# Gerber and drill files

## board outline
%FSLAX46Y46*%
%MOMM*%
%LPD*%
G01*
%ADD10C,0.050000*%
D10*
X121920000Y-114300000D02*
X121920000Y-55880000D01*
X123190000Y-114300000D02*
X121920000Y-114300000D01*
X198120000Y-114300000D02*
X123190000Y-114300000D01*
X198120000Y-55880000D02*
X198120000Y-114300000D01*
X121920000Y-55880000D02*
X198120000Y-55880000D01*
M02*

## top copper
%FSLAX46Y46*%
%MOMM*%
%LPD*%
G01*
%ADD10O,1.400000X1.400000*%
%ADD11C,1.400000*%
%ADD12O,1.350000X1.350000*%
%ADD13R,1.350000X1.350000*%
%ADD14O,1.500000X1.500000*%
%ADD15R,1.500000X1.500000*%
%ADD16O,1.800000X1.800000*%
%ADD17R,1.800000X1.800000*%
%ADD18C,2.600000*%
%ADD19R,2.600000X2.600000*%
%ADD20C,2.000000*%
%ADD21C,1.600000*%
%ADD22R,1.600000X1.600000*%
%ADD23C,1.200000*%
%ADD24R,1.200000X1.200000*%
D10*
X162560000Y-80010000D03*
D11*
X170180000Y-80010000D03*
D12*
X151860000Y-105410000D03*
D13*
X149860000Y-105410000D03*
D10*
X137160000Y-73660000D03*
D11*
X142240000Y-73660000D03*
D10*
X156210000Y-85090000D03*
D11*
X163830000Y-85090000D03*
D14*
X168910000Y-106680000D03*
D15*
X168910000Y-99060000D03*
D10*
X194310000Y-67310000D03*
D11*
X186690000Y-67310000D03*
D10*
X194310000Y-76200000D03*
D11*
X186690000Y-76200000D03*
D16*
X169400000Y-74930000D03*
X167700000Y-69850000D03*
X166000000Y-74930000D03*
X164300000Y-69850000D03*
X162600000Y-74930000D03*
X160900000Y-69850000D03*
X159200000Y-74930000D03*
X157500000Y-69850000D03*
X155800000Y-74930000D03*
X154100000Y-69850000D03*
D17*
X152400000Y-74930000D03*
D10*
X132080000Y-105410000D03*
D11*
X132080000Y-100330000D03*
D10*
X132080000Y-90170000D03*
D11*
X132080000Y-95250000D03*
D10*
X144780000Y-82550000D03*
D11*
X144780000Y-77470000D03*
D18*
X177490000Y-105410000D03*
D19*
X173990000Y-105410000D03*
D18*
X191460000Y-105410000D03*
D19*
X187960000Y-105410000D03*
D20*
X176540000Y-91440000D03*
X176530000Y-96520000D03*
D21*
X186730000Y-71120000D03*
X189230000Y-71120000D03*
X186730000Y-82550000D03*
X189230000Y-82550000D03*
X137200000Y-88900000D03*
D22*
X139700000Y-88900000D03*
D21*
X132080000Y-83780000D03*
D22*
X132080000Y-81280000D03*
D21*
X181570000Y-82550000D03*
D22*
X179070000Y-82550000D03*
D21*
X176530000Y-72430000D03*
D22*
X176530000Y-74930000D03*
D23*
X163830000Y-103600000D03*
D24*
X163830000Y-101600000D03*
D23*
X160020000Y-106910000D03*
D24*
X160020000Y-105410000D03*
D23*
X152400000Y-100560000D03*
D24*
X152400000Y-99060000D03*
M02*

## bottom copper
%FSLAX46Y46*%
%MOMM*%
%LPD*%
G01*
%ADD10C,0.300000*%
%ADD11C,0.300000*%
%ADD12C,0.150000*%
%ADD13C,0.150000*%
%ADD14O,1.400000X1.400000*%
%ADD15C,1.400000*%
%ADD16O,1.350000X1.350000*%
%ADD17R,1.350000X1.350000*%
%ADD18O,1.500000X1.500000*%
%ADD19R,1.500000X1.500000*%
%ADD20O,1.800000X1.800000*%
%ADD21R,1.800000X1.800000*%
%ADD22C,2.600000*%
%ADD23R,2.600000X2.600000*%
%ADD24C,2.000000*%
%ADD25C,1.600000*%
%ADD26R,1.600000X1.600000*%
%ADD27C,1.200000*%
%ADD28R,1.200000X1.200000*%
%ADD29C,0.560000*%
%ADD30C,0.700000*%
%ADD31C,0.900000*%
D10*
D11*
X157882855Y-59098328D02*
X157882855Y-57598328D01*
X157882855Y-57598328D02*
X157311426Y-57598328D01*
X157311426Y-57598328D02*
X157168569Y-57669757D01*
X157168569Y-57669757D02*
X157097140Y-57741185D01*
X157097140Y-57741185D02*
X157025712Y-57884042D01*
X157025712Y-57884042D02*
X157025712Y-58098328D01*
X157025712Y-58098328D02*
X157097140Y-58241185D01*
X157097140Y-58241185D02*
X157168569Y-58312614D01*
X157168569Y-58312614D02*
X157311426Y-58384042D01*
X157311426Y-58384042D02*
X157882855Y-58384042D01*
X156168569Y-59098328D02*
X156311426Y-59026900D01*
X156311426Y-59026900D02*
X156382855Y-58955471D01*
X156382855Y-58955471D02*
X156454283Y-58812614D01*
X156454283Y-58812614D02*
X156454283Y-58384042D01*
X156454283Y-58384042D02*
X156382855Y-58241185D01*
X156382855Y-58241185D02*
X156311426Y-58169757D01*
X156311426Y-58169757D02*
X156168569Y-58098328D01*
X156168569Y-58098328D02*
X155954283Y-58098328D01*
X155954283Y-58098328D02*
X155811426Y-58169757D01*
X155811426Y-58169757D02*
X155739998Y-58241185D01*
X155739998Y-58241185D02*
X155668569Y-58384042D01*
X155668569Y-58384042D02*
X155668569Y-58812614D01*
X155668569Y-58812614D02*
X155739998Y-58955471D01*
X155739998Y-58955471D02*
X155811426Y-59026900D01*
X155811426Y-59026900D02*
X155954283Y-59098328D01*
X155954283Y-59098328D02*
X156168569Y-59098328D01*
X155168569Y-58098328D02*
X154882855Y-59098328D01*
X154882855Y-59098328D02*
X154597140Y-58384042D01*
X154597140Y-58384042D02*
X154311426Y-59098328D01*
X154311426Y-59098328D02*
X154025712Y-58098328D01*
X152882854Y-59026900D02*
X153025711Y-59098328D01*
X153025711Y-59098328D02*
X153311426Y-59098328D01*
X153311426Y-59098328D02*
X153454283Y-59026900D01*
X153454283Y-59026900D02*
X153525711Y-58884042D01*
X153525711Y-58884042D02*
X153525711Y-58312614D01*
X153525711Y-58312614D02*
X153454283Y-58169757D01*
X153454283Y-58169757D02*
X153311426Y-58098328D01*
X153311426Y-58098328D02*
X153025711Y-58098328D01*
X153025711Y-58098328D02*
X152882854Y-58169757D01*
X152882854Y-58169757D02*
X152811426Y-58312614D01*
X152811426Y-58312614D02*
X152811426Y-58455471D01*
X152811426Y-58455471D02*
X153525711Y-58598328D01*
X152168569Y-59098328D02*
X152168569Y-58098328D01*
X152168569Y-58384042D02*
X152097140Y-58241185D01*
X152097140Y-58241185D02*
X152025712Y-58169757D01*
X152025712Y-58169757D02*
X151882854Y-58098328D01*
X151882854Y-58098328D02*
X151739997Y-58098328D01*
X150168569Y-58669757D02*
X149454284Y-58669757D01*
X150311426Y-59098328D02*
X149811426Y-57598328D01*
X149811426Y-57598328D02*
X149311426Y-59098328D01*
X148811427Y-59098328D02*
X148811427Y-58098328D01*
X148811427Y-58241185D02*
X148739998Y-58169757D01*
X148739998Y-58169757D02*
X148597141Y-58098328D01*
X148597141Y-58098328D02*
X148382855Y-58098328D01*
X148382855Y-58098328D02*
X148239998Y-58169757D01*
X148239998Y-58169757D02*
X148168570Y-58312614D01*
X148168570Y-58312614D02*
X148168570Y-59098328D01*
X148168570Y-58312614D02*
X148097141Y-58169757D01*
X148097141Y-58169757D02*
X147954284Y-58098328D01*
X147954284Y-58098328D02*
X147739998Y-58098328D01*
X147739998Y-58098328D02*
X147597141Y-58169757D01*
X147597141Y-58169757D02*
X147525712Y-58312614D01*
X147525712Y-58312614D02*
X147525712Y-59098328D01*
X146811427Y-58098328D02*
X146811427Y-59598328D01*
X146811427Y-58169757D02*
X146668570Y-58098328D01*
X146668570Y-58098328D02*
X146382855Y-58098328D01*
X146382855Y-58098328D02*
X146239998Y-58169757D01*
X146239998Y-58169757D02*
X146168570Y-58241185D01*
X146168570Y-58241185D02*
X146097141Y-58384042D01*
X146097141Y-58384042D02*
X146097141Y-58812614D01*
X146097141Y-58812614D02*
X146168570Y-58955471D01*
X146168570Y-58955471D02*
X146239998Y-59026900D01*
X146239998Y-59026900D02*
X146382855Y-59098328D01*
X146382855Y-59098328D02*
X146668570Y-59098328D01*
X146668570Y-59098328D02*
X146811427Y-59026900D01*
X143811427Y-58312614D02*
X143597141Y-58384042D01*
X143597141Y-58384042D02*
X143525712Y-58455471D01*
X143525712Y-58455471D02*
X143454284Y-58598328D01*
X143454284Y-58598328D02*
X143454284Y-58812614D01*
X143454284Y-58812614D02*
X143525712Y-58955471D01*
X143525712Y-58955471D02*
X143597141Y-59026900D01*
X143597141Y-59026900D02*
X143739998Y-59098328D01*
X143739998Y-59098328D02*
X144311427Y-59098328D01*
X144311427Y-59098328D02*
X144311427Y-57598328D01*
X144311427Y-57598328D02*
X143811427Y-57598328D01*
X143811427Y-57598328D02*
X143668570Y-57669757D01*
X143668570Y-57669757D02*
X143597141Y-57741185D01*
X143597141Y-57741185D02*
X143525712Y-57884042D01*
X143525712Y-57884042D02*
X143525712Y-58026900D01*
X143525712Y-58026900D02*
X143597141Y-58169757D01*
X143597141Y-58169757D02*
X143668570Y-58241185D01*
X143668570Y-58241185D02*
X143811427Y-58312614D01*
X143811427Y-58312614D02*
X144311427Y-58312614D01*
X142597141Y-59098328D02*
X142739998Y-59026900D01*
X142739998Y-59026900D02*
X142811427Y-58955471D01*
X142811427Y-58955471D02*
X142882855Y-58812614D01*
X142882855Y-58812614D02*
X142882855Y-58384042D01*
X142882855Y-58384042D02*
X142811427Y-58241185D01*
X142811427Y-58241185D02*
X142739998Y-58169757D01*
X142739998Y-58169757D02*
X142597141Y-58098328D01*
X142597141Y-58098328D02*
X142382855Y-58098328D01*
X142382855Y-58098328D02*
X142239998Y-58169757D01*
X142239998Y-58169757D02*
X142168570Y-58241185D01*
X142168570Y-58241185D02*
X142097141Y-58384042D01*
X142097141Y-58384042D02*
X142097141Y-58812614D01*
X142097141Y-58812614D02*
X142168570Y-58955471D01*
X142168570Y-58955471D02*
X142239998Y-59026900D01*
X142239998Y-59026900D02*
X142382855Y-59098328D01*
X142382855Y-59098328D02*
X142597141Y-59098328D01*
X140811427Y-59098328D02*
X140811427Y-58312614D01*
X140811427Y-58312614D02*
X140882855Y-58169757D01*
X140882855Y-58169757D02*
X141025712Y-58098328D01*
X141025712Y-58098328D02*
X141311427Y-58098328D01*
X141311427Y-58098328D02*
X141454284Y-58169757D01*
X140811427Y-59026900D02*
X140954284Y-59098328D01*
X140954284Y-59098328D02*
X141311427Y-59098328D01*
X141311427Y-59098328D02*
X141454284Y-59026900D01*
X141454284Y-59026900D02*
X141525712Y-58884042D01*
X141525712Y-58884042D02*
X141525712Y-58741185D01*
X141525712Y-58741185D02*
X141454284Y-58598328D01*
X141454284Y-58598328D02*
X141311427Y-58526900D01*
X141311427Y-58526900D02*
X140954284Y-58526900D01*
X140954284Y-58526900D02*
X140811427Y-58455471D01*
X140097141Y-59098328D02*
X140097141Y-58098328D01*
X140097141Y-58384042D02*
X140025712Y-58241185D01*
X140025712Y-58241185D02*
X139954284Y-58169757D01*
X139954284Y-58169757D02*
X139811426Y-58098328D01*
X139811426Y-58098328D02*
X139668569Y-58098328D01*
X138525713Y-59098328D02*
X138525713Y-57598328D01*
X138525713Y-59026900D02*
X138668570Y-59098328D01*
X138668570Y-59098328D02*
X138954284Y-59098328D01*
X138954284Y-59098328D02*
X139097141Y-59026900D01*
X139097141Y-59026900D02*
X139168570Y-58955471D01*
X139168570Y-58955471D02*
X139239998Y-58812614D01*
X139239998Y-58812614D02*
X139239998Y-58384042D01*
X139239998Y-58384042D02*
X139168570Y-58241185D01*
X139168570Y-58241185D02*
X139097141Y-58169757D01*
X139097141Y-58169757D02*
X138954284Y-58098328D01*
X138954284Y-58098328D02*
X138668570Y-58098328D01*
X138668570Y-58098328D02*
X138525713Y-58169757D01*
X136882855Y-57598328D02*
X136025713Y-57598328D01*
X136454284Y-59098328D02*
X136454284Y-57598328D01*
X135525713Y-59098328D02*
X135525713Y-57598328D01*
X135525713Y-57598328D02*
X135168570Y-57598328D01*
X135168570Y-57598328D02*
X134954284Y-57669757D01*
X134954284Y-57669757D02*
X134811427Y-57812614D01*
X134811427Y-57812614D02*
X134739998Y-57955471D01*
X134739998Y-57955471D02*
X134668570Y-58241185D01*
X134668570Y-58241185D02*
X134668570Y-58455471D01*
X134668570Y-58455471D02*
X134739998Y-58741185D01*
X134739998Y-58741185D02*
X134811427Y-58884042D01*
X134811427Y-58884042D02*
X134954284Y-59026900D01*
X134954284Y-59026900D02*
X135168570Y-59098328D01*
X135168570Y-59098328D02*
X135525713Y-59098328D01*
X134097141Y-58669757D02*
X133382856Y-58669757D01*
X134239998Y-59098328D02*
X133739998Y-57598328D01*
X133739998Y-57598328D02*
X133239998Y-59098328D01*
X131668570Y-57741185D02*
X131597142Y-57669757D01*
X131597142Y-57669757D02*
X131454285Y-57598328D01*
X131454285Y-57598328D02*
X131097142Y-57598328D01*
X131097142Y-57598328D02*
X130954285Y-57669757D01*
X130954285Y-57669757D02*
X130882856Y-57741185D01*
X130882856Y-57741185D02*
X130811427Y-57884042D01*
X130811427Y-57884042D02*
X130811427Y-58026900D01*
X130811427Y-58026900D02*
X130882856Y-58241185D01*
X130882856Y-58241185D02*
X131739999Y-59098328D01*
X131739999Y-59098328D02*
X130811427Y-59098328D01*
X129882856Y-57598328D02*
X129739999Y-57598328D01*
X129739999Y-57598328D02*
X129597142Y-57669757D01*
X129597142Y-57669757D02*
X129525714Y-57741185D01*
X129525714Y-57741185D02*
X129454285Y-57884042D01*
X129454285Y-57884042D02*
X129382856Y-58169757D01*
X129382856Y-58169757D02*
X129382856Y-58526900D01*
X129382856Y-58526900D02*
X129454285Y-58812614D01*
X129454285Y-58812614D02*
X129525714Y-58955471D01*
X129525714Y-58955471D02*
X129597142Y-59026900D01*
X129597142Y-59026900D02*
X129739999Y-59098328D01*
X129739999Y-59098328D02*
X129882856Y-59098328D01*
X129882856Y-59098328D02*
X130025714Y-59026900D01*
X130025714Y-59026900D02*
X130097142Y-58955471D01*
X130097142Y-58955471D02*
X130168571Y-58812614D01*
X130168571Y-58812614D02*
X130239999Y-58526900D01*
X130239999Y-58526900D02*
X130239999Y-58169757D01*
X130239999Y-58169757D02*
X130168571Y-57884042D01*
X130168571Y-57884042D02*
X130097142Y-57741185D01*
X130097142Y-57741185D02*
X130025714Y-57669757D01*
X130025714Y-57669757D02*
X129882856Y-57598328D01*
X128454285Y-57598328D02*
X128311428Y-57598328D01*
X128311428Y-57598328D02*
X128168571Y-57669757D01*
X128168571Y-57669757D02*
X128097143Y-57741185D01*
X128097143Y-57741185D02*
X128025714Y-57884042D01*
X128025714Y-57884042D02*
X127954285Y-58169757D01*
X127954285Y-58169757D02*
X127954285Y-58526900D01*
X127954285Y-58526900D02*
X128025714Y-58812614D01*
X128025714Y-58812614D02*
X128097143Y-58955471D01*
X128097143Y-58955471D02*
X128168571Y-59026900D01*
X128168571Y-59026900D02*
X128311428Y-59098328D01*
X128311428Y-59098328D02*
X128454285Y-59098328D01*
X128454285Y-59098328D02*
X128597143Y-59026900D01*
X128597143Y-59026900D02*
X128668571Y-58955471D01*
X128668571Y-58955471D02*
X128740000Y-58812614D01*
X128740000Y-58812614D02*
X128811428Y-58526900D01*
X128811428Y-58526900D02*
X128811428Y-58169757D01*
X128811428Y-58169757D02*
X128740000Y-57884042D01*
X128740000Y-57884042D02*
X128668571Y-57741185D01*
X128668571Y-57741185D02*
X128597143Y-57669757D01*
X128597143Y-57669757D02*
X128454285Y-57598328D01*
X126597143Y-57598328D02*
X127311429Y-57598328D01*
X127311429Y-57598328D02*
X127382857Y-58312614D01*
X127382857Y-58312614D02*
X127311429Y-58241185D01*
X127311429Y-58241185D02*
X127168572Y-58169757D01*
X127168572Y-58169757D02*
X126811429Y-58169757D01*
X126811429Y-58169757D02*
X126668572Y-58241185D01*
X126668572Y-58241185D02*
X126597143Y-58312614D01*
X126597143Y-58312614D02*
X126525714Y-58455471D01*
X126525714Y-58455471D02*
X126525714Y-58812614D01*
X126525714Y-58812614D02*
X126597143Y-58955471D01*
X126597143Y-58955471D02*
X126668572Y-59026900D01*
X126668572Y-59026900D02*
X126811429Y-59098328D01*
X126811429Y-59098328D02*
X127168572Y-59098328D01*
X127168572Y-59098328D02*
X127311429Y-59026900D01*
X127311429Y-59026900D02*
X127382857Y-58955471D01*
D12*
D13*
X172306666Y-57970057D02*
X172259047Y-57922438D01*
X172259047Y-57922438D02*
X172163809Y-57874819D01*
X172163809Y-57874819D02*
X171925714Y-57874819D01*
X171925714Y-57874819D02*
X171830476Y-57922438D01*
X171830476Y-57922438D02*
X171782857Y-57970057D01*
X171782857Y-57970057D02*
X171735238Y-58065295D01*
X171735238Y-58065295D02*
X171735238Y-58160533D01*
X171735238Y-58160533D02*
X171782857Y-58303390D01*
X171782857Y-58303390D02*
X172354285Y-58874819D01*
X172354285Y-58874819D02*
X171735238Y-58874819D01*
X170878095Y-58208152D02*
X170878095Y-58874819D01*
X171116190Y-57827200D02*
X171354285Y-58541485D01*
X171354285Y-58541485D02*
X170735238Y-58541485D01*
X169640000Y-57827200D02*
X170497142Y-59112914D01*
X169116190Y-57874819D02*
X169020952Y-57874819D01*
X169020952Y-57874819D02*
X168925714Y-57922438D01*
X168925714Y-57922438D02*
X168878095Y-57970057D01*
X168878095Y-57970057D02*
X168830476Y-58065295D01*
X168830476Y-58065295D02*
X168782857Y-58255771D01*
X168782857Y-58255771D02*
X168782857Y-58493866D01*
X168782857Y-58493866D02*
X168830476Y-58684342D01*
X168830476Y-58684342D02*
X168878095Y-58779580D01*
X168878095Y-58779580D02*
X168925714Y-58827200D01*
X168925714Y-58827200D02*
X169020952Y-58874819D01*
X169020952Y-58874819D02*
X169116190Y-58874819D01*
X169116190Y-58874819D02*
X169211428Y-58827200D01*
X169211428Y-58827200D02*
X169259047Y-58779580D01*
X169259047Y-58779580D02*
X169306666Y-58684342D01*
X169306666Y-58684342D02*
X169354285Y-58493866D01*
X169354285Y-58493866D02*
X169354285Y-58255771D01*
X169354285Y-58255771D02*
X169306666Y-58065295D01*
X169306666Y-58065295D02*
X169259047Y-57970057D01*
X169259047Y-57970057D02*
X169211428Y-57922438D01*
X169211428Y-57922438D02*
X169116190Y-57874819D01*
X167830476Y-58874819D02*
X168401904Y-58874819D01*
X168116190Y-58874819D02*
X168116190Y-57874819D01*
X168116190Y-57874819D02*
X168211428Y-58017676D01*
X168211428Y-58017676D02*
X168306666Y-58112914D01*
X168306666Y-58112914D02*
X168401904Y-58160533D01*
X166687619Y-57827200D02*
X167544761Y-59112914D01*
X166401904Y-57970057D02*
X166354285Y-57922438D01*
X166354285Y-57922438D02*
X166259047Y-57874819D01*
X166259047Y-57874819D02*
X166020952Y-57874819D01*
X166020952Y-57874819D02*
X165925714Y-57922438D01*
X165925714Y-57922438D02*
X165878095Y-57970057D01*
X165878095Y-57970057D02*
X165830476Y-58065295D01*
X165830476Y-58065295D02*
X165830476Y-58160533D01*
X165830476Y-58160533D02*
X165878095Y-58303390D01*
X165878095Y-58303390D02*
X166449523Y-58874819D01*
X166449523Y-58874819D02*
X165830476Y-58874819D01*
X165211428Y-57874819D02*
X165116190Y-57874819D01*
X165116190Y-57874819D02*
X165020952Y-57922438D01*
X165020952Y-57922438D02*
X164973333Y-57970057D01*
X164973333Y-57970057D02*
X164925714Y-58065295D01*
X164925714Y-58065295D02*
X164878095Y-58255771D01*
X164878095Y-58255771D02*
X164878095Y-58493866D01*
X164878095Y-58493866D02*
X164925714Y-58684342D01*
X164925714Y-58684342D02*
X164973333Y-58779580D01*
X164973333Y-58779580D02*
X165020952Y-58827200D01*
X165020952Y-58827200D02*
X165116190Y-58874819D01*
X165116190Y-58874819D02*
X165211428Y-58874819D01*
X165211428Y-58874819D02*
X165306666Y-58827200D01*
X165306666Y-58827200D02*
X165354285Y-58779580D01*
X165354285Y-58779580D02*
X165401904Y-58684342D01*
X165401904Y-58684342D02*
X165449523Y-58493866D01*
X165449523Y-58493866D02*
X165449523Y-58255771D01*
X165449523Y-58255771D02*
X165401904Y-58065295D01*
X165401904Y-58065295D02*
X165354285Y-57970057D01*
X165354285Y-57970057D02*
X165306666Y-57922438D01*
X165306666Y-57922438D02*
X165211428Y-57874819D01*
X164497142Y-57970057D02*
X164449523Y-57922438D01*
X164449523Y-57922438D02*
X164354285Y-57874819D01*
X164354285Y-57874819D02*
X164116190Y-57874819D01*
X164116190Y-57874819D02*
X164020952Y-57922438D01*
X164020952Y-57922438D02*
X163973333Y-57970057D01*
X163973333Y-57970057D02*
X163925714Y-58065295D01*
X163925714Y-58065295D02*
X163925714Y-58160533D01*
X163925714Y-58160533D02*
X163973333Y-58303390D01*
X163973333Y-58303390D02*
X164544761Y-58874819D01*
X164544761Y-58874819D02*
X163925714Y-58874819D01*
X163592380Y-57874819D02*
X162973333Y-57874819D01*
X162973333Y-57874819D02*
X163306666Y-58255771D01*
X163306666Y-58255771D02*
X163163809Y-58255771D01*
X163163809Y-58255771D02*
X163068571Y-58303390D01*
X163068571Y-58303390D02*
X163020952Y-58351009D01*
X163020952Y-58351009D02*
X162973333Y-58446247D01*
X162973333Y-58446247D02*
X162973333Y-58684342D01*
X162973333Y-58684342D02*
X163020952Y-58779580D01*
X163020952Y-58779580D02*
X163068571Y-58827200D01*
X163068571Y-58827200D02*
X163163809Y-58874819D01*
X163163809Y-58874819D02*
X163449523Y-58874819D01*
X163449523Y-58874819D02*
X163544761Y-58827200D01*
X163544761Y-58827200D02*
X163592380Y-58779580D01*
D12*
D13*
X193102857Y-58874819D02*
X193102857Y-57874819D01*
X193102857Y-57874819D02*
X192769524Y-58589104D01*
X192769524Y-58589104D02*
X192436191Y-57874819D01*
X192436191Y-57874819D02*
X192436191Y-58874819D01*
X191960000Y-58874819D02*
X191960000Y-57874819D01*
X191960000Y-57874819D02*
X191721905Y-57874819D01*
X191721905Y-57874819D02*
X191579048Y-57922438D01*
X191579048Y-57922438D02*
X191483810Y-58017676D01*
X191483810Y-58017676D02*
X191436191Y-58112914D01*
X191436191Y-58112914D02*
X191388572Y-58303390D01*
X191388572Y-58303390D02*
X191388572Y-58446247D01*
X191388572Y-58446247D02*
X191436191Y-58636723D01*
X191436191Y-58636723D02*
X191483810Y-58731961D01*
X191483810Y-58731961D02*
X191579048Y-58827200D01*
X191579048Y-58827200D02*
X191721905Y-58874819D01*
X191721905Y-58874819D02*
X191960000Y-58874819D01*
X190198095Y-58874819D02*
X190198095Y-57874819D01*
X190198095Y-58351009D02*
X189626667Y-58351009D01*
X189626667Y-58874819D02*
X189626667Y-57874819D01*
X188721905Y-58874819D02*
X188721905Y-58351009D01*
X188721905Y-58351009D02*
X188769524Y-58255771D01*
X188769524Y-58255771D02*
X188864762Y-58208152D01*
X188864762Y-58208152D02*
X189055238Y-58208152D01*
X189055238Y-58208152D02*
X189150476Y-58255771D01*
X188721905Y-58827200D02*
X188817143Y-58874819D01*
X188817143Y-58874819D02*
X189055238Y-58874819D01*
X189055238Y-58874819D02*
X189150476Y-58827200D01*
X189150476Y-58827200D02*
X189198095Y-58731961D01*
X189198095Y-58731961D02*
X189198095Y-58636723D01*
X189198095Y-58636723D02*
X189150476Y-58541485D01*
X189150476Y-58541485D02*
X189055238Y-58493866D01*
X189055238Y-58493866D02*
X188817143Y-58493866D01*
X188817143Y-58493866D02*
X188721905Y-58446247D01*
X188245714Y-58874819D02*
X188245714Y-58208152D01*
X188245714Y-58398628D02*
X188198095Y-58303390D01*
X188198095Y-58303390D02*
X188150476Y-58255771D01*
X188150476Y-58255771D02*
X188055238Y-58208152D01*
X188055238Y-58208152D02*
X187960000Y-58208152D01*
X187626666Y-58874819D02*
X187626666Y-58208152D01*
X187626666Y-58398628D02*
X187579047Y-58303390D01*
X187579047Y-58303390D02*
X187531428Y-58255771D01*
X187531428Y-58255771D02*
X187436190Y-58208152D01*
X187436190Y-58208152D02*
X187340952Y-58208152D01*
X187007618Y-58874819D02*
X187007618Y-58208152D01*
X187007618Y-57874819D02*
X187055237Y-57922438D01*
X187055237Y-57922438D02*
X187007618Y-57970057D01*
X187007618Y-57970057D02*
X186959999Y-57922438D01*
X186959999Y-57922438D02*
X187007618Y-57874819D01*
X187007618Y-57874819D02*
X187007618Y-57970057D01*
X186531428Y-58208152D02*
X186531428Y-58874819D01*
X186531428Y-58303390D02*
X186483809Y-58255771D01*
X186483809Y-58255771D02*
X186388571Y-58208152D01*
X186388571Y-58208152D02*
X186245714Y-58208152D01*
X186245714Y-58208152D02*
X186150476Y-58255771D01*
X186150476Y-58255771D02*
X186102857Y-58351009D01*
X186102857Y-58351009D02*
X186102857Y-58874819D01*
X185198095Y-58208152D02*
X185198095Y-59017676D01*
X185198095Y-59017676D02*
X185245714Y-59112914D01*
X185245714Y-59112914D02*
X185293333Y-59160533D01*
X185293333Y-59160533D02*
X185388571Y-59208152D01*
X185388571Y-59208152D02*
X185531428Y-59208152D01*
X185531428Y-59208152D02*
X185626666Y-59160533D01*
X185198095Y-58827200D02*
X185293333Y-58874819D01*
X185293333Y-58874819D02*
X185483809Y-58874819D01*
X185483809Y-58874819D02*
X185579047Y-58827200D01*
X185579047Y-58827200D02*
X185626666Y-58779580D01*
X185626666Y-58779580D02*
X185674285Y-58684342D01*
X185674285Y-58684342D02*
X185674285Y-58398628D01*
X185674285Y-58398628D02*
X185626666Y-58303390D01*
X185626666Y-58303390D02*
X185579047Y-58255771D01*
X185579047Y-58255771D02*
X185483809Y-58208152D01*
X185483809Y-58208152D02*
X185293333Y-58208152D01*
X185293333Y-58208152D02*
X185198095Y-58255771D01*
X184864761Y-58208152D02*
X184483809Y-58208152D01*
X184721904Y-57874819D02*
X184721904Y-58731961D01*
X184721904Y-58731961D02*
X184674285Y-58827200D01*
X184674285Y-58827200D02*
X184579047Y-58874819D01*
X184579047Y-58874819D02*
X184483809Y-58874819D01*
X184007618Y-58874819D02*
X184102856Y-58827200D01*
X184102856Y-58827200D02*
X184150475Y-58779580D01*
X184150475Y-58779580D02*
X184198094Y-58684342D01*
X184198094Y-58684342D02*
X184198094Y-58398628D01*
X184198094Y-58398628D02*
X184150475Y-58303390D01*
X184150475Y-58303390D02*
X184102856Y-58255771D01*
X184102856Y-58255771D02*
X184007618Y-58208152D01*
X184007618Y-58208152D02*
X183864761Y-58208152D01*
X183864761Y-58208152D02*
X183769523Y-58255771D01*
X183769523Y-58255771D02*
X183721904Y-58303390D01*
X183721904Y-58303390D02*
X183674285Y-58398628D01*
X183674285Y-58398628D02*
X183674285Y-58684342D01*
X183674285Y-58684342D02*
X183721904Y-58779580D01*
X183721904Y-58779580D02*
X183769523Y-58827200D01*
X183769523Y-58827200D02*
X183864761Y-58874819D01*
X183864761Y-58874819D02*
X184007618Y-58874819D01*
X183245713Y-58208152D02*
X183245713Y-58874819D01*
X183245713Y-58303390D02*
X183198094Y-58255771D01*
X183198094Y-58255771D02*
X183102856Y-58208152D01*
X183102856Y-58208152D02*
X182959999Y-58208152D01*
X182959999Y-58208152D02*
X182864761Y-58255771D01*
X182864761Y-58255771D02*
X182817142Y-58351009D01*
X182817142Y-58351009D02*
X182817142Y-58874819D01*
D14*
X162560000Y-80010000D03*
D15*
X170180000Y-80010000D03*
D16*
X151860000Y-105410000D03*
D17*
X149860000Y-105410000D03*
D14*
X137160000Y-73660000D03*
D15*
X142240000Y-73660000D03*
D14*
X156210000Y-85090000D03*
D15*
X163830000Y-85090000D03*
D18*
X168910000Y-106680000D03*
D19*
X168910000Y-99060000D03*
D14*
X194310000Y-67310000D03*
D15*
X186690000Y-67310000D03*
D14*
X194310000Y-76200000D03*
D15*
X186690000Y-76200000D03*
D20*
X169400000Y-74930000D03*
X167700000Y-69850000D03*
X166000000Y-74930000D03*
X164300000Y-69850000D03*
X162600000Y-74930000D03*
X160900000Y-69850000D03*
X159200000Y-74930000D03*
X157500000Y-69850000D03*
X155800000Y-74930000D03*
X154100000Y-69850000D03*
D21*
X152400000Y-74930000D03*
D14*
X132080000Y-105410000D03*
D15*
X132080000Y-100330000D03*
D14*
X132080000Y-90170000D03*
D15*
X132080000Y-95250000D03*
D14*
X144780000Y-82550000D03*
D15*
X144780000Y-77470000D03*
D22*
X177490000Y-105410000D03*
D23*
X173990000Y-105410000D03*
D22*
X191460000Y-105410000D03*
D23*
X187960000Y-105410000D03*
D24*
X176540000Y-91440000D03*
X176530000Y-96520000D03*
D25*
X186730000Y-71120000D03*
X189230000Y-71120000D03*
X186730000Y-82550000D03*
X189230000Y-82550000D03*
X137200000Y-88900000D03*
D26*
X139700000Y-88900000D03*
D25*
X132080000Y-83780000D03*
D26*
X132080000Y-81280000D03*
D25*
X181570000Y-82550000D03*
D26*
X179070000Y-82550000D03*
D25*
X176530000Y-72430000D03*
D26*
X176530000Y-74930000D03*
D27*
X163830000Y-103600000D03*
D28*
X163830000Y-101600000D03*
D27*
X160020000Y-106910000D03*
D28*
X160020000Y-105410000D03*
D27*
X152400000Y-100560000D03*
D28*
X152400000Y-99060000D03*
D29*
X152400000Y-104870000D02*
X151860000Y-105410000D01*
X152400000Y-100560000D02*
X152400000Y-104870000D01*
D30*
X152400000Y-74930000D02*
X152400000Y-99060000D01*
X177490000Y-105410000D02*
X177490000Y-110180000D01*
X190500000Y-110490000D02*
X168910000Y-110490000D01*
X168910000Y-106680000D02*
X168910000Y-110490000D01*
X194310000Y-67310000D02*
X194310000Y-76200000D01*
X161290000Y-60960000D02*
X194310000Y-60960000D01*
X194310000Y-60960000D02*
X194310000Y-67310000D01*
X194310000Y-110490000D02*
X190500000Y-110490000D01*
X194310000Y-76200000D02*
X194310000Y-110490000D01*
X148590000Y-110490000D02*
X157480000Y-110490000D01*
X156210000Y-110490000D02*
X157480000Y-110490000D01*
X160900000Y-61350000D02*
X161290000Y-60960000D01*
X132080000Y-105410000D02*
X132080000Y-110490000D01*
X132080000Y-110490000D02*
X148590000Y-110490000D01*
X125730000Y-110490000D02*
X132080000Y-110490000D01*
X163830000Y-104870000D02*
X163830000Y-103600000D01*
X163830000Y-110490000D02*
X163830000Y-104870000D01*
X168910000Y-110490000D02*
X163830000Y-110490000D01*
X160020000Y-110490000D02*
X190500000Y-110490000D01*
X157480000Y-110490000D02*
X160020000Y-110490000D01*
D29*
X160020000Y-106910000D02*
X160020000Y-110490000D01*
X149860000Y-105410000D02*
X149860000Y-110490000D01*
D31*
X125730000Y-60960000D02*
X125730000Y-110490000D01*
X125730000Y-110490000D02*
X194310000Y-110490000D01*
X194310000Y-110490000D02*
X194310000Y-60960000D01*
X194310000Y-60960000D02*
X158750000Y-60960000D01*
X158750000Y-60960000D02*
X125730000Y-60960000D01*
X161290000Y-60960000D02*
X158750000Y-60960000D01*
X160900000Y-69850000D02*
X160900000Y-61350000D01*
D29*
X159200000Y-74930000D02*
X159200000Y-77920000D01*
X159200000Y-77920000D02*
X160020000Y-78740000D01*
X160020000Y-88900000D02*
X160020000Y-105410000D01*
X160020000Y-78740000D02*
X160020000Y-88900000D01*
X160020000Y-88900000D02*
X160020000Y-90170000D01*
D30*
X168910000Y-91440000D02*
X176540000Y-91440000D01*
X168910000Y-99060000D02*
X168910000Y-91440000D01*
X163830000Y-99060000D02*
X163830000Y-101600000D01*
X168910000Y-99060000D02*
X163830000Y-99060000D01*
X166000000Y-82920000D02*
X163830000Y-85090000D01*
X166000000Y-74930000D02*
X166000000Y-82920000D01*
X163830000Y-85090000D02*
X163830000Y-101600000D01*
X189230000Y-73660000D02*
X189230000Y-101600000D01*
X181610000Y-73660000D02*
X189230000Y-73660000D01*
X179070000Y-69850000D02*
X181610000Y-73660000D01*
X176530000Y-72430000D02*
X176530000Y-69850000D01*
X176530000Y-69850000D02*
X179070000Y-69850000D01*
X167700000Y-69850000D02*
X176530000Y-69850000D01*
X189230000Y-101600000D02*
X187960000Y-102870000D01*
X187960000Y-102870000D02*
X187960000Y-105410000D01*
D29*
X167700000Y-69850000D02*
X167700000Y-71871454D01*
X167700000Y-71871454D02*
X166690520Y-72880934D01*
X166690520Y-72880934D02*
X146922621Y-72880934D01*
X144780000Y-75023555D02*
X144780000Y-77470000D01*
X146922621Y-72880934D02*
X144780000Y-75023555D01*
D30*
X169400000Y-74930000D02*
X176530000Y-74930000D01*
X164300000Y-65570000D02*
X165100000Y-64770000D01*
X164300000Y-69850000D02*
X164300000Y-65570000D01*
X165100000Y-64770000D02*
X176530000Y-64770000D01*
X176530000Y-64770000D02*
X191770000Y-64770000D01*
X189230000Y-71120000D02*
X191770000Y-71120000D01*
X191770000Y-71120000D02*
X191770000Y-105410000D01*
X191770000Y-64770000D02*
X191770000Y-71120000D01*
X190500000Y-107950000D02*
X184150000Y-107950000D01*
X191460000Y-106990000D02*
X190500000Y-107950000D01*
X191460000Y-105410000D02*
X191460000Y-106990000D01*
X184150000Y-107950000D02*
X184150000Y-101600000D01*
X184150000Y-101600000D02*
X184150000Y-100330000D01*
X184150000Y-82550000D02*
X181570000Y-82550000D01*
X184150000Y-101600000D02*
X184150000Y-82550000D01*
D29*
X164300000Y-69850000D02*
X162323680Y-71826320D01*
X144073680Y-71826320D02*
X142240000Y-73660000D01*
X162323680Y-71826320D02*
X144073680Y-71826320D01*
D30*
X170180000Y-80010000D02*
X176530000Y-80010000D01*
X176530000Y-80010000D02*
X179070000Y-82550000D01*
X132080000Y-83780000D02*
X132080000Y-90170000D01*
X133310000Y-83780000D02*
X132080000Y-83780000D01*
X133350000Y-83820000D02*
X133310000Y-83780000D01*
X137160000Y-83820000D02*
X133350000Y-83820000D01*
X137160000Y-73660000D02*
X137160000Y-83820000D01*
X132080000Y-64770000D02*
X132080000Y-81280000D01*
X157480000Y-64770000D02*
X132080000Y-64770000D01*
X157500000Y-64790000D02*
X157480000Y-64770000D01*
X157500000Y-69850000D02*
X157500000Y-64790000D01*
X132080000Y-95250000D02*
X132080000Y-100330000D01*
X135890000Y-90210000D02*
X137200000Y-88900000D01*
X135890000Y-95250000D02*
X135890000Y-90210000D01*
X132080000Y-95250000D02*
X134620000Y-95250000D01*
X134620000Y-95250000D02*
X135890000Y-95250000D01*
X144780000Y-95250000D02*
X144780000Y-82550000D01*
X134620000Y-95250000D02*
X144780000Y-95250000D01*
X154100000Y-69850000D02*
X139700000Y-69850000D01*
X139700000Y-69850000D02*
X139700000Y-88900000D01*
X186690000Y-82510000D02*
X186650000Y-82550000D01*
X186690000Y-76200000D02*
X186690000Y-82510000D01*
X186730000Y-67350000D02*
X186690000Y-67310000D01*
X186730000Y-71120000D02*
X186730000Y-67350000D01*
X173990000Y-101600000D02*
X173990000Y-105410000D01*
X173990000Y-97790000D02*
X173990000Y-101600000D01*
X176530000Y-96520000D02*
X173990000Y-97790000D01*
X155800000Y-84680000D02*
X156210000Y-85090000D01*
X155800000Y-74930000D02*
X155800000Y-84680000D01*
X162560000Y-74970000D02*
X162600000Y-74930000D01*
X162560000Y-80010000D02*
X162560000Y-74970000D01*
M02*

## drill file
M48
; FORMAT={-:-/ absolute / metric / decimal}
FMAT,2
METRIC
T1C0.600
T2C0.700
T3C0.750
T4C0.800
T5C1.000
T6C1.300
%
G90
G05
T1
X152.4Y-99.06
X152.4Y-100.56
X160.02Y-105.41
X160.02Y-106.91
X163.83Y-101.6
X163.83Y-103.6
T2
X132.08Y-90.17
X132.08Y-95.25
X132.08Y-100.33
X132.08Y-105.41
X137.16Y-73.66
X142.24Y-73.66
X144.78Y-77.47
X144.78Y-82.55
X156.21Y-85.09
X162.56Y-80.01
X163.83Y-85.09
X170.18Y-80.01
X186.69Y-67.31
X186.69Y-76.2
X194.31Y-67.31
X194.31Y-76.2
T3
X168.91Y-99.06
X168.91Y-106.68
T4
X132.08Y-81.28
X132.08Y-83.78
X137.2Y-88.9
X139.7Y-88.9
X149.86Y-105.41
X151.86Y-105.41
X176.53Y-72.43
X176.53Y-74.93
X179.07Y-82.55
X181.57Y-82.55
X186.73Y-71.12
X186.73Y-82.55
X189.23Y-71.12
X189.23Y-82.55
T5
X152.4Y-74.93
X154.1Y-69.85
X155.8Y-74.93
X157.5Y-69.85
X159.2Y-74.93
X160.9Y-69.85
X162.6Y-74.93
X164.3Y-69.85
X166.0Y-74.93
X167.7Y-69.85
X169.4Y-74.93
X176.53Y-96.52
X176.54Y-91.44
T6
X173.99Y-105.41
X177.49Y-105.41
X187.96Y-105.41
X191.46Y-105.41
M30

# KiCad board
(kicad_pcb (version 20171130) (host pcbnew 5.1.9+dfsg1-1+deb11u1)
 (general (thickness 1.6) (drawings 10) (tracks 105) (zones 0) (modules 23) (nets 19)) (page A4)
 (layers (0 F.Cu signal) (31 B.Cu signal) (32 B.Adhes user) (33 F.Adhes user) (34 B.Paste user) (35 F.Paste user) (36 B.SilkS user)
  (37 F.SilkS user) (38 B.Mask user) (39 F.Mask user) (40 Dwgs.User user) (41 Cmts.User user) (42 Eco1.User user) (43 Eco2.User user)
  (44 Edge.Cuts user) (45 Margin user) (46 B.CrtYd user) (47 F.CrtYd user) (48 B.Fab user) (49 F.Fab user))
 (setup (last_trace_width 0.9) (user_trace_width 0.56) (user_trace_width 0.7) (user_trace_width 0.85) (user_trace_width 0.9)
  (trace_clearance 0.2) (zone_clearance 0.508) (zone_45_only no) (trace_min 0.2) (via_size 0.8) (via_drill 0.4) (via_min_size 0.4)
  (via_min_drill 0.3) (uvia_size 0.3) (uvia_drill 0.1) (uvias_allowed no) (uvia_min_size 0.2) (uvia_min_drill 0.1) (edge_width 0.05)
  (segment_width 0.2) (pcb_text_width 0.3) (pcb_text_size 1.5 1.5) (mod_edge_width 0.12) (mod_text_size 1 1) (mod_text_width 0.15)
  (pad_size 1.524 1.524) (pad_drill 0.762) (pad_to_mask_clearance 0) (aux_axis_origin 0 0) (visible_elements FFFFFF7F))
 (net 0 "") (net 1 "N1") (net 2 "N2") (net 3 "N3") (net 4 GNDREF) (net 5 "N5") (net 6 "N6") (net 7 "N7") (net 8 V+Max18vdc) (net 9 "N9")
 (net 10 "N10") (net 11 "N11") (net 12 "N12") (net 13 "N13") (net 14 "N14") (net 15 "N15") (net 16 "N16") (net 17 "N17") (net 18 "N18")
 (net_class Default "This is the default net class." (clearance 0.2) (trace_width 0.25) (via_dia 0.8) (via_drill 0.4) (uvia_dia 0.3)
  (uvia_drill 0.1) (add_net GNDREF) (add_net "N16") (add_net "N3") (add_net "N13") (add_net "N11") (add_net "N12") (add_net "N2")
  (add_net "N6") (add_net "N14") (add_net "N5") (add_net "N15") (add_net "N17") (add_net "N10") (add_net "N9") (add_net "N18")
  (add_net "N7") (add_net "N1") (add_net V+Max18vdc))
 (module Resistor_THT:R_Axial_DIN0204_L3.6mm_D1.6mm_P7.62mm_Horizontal (layer F.Cu) (at 170.18 80.01 180)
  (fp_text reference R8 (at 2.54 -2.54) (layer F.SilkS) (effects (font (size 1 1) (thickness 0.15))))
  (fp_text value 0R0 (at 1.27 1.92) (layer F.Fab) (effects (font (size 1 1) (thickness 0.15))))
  (pad 2 thru_hole oval (at 7.62 0 180) (size 1.4 1.4) (drill 0.7) (layers *.Cu *.Mask) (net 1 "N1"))
  (pad 1 thru_hole circle (at 0 0 180) (size 1.4 1.4) (drill 0.7) (layers *.Cu *.Mask) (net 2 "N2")))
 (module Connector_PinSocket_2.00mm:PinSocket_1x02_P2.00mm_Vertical (layer F.Cu) (at 149.86 105.41 90)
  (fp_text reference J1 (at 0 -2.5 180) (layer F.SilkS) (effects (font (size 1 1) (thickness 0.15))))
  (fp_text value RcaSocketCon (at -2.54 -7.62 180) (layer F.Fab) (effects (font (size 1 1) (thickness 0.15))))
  (pad 2 thru_hole oval (at 0 2 90) (size 1.35 1.35) (drill 0.8) (layers *.Cu *.Mask) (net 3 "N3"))
  (pad 1 thru_hole rect (at 0 0 90) (size 1.35 1.35) (drill 0.8) (layers *.Cu *.Mask) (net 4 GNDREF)))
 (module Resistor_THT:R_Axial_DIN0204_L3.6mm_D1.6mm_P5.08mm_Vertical (layer F.Cu) (at 142.24 73.66 180)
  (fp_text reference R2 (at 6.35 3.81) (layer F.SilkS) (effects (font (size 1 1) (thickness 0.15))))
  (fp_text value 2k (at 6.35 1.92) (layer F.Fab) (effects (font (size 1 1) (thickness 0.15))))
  (pad 2 thru_hole oval (at 5.08 0 180) (size 1.4 1.4) (drill 0.7) (layers *.Cu *.Mask) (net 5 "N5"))
  (pad 1 thru_hole circle (at 0 0 180) (size 1.4 1.4) (drill 0.7) (layers *.Cu *.Mask) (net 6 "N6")))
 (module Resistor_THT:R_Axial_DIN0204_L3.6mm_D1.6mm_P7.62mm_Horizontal (layer F.Cu) (at 163.83 85.09 180)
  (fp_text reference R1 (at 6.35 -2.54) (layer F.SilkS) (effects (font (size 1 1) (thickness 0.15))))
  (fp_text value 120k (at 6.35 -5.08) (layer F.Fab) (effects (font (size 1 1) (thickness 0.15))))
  (pad 2 thru_hole oval (at 7.62 0 180) (size 1.4 1.4) (drill 0.7) (layers *.Cu *.Mask) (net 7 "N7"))
  (pad 1 thru_hole circle (at 0 0 180) (size 1.4 1.4) (drill 0.7) (layers *.Cu *.Mask) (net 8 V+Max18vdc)))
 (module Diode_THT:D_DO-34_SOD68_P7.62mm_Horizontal (layer F.Cu) (at 168.91 99.06 270)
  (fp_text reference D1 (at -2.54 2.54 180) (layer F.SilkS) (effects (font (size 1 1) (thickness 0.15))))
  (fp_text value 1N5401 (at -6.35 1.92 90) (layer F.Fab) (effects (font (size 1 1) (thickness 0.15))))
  (pad 2 thru_hole oval (at 7.62 0 270) (size 1.5 1.5) (drill 0.75) (layers *.Cu *.Mask) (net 4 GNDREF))
  (pad 1 thru_hole rect (at 0 0 270) (size 1.5 1.5) (drill 0.75) (layers *.Cu *.Mask) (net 8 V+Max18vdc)))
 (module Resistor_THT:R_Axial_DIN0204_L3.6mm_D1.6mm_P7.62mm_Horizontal (layer F.Cu) (at 186.69 67.31)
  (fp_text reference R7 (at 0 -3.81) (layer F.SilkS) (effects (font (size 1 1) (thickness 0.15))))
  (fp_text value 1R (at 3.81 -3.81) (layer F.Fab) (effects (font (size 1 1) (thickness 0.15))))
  (pad 2 thru_hole oval (at 7.62 0) (size 1.4 1.4) (drill 0.7) (layers *.Cu *.Mask) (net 4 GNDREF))
  (pad 1 thru_hole circle (at 0 0) (size 1.4 1.4) (drill 0.7) (layers *.Cu *.Mask) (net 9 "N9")))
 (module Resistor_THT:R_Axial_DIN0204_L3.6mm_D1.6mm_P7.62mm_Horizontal (layer F.Cu) (at 186.69 76.2)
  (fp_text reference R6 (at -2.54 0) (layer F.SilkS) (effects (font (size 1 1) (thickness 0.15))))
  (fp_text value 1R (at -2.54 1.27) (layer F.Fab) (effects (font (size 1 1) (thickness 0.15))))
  (pad 2 thru_hole oval (at 7.62 0) (size 1.4 1.4) (drill 0.7) (layers *.Cu *.Mask) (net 4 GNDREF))
  (pad 1 thru_hole circle (at 0 0) (size 1.4 1.4) (drill 0.7) (layers *.Cu *.Mask) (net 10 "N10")))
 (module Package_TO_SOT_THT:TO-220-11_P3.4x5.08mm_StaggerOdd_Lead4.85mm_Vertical (layer F.Cu) (at 152.4 74.93)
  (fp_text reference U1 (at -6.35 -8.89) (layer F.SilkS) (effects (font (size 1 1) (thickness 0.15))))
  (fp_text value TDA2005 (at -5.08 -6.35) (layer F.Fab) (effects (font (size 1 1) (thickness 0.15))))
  (pad 11 thru_hole oval (at 17 0) (size 1.8 1.8) (drill 1) (layers *.Cu *.Mask) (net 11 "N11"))
  (pad 10 thru_hole oval (at 15.3 -5.08) (size 1.8 1.8) (drill 1) (layers *.Cu *.Mask) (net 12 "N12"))
  (pad 9 thru_hole oval (at 13.6 0) (size 1.8 1.8) (drill 1) (layers *.Cu *.Mask) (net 8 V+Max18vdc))
  (pad 8 thru_hole oval (at 11.9 -5.08) (size 1.8 1.8) (drill 1) (layers *.Cu *.Mask) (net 6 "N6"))
  (pad 7 thru_hole oval (at 10.2 0) (size 1.8 1.8) (drill 1) (layers *.Cu *.Mask) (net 1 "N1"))
  (pad 6 thru_hole oval (at 8.5 -5.08) (size 1.8 1.8) (drill 1) (layers *.Cu *.Mask) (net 4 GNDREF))
  (pad 5 thru_hole oval (at 6.8 0) (size 1.8 1.8) (drill 1) (layers *.Cu *.Mask) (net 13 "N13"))
  (pad 4 thru_hole oval (at 5.1 -5.08) (size 1.8 1.8) (drill 1) (layers *.Cu *.Mask) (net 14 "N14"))
  (pad 3 thru_hole oval (at 3.4 0) (size 1.8 1.8) (drill 1) (layers *.Cu *.Mask) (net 7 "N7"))
  (pad 2 thru_hole oval (at 1.7 -5.08) (size 1.8 1.8) (drill 1) (layers *.Cu *.Mask) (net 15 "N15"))
  (pad 1 thru_hole rect (at 0 0) (size 1.8 1.8) (drill 1) (layers *.Cu *.Mask) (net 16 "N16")))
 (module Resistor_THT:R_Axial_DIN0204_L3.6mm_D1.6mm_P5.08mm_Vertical (layer F.Cu) (at 132.08 100.33 270)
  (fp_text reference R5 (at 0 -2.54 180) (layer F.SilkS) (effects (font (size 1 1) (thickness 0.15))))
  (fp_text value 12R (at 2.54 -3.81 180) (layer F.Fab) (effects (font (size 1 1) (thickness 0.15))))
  (pad 2 thru_hole oval (at 5.08 0 270) (size 1.4 1.4) (drill 0.7) (layers *.Cu *.Mask) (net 4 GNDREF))
  (pad 1 thru_hole circle (at 0 0 270) (size 1.4 1.4) (drill 0.7) (layers *.Cu *.Mask) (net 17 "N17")))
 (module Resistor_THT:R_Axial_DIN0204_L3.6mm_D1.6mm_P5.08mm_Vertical (layer F.Cu) (at 132.08 95.25 90)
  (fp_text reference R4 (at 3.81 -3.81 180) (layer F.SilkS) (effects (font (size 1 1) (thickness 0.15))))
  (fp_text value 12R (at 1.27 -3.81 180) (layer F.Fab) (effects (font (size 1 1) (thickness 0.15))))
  (pad 2 thru_hole oval (at 5.08 0 90) (size 1.4 1.4) (drill 0.7) (layers *.Cu *.Mask) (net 5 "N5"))
  (pad 1 thru_hole circle (at 0 0 90) (size 1.4 1.4) (drill 0.7) (layers *.Cu *.Mask) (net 17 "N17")))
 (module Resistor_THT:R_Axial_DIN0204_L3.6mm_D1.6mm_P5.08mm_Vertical (layer F.Cu) (at 144.78 77.47 270)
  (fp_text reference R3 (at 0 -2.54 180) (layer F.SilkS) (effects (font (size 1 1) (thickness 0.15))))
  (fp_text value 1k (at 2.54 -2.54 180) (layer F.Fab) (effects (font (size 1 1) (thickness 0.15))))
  (pad 2 thru_hole oval (at 5.08 0 270) (size 1.4 1.4) (drill 0.7) (layers *.Cu *.Mask) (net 17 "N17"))
  (pad 1 thru_hole circle (at 0 0 270) (size 1.4 1.4) (drill 0.7) (layers *.Cu *.Mask) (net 12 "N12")))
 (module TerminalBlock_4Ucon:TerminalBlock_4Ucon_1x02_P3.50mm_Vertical (layer F.Cu) (at 173.99 105.41)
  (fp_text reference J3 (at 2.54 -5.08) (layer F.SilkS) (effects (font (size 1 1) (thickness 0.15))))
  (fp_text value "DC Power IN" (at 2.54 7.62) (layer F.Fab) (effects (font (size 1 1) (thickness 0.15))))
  (pad 2 thru_hole circle (at 3.5 0) (size 2.6 2.6) (drill 1.3) (layers *.Cu *.Mask) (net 4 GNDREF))
  (pad 1 thru_hole rect (at 0 0) (size 2.6 2.6) (drill 1.3) (layers *.Cu *.Mask) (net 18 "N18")))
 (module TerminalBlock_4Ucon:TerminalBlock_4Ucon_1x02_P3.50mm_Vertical (layer F.Cu) (at 187.96 105.41)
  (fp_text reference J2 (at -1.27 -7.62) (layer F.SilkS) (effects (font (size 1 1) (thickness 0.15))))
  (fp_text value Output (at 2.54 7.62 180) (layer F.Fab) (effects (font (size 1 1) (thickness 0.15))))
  (pad 2 thru_hole circle (at 3.5 0) (size 2.6 2.6) (drill 1.3) (layers *.Cu *.Mask) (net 6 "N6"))
  (pad 1 thru_hole rect (at 0 0) (size 2.6 2.6) (drill 1.3) (layers *.Cu *.Mask) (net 12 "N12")))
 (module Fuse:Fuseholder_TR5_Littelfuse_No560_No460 (layer F.Cu) (at 176.53 96.52 90)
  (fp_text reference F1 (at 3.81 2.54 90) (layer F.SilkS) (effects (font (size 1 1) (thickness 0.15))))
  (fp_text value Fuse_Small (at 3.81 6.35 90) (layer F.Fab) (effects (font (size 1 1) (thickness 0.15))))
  (pad 2 thru_hole circle (at 5.08 0.01 90) (size 2 2) (drill 1) (layers *.Cu *.Mask) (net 8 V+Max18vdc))
  (pad 1 thru_hole circle (at 0 0 90) (size 2 2) (drill 1) (layers *.Cu *.Mask) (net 18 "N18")))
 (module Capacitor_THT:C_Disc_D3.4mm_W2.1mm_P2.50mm (layer F.Cu) (at 189.23 71.12 180)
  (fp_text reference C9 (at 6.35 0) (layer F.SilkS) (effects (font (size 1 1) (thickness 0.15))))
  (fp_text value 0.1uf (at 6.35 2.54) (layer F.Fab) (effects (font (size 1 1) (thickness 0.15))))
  (pad 2 thru_hole circle (at 2.5 0 180) (size 1.6 1.6) (drill 0.8) (layers *.Cu *.Mask) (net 9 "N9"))
  (pad 1 thru_hole circle (at 0 0 180) (size 1.6 1.6) (drill 0.8) (layers *.Cu *.Mask) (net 6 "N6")))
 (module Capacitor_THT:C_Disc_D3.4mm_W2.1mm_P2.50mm (layer F.Cu) (at 189.23 82.55 180)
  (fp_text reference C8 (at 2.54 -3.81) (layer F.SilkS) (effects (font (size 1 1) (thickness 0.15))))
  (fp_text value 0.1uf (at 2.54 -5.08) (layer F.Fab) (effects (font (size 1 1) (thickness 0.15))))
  (pad 2 thru_hole circle (at 2.5 0 180) (size 1.6 1.6) (drill 0.8) (layers *.Cu *.Mask) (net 10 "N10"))
  (pad 1 thru_hole circle (at 0 0 180) (size 1.6 1.6) (drill 0.8) (layers *.Cu *.Mask) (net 12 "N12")))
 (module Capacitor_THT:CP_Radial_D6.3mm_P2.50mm (layer F.Cu) (at 139.7 88.9 180)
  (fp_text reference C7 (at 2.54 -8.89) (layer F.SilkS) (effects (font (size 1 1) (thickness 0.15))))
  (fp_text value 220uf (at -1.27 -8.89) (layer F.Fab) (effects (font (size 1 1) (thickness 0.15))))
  (pad 2 thru_hole circle (at 2.5 0 180) (size 1.6 1.6) (drill 0.8) (layers *.Cu *.Mask) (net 17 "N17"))
  (pad 1 thru_hole rect (at 0 0 180) (size 1.6 1.6) (drill 0.8) (layers *.Cu *.Mask) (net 15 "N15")))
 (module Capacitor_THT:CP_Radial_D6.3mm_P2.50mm (layer F.Cu) (at 132.08 81.28 270)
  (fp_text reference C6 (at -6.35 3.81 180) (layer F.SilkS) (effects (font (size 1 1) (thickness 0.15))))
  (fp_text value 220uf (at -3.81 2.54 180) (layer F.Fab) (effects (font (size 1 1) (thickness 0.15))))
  (pad 2 thru_hole circle (at 2.5 0 270) (size 1.6 1.6) (drill 0.8) (layers *.Cu *.Mask) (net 5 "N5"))
  (pad 1 thru_hole rect (at 0 0 270) (size 1.6 1.6) (drill 0.8) (layers *.Cu *.Mask) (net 14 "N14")))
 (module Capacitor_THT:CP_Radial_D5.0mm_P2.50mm (layer F.Cu) (at 179.07 82.55)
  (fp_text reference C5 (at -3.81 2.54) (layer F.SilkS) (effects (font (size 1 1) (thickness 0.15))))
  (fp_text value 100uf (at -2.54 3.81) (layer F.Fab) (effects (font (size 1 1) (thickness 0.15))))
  (pad 2 thru_hole circle (at 2.5 0) (size 1.6 1.6) (drill 0.8) (layers *.Cu *.Mask) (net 6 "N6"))
  (pad 1 thru_hole rect (at 0 0) (size 1.6 1.6) (drill 0.8) (layers *.Cu *.Mask) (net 2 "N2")))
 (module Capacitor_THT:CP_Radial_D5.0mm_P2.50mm (layer F.Cu) (at 176.53 74.93 90)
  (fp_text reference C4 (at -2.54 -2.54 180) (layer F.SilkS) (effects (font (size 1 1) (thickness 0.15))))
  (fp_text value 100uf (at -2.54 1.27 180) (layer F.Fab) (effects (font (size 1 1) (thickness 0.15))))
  (pad 2 thru_hole circle (at 2.5 0 90) (size 1.6 1.6) (drill 0.8) (layers *.Cu *.Mask) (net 12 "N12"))
  (pad 1 thru_hole rect (at 0 0 90) (size 1.6 1.6) (drill 0.8) (layers *.Cu *.Mask) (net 11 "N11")))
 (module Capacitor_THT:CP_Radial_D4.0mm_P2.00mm (layer F.Cu) (at 163.83 101.6 270)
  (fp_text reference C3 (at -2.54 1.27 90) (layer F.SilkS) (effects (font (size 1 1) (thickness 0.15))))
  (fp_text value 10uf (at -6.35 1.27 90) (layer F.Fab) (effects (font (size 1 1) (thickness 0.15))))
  (pad 2 thru_hole circle (at 2 0 270) (size 1.2 1.2) (drill 0.6) (layers *.Cu *.Mask) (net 4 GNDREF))
  (pad 1 thru_hole rect (at 0 0 270) (size 1.2 1.2) (drill 0.6) (layers *.Cu *.Mask) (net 8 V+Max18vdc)))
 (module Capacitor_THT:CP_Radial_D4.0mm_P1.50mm (layer F.Cu) (at 160.02 105.41 270)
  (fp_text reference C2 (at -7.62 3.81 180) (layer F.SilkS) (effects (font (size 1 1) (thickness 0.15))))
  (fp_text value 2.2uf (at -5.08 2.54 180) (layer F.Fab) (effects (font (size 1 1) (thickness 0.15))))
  (pad 2 thru_hole circle (at 1.5 0 270) (size 1.2 1.2) (drill 0.6) (layers *.Cu *.Mask) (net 4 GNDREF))
  (pad 1 thru_hole rect (at 0 0 270) (size 1.2 1.2) (drill 0.6) (layers *.Cu *.Mask) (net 13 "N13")))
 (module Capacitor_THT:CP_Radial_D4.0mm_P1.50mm (layer F.Cu) (at 152.4 99.06 270)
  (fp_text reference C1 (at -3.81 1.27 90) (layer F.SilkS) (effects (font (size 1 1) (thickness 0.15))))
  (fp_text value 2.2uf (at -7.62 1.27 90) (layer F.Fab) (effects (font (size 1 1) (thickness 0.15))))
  (pad 2 thru_hole circle (at 1.5 0 270) (size 1.2 1.2) (drill 0.6) (layers *.Cu *.Mask) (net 3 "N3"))
  (pad 1 thru_hole rect (at 0 0 270) (size 1.2 1.2) (drill 0.6) (layers *.Cu *.Mask) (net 16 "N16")))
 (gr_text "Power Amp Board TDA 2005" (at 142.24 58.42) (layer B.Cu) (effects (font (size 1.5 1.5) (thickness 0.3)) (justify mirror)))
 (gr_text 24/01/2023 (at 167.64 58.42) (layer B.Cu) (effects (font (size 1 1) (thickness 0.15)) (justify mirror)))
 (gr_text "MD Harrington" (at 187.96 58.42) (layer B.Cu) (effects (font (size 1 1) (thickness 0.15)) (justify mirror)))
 (gr_line (start 121.92 114.3) (end 121.92 55.88) (layer Edge.Cuts) (width 0.05))
 (gr_line (start 123.19 114.3) (end 121.92 114.3) (layer Edge.Cuts) (width 0.05))
 (gr_line (start 198.12 114.3) (end 123.19 114.3) (layer Edge.Cuts) (width 0.05))
 (gr_line (start 198.12 55.88) (end 198.12 114.3) (layer Edge.Cuts) (width 0.05))
 (gr_line (start 121.92 55.88) (end 198.12 55.88) (layer Edge.Cuts) (width 0.05))
 (segment (start 152.4 104.87) (end 151.86 105.41) (width 0.56) (layer B.Cu) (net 3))
 (segment (start 152.4 100.56) (end 152.4 104.87) (width 0.56) (layer B.Cu) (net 3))
 (segment (start 152.4 74.93) (end 152.4 99.06) (width 0.7) (layer B.Cu) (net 16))
 (segment (start 177.49 105.41) (end 177.49 110.18) (width 0.7) (layer B.Cu) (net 4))
 (segment (start 190.5 110.49) (end 168.91 110.49) (width 0.7) (layer B.Cu) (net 4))
 (segment (start 168.91 106.68) (end 168.91 110.49) (width 0.7) (layer B.Cu) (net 4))
 (segment (start 194.31 67.31) (end 194.31 76.2) (width 0.7) (layer B.Cu) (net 4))
 (segment (start 161.29 60.96) (end 194.31 60.96) (width 0.7) (layer B.Cu) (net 4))
 (segment (start 194.31 60.96) (end 194.31 67.31) (width 0.7) (layer B.Cu) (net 4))
 (segment (start 194.31 110.49) (end 190.5 110.49) (width 0.7) (layer B.Cu) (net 4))
 (segment (start 194.31 76.2) (end 194.31 110.49) (width 0.7) (layer B.Cu) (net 4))
 (segment (start 148.59 110.49) (end 157.48 110.49) (width 0.7) (layer B.Cu) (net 4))
 (segment (start 156.21 110.49) (end 157.48 110.49) (width 0.7) (layer B.Cu) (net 4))
 (segment (start 160.9 61.35) (end 161.29 60.96) (width 0.7) (layer B.Cu) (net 4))
 (segment (start 132.08 105.41) (end 132.08 110.49) (width 0.7) (layer B.Cu) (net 4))
 (segment (start 132.08 110.49) (end 148.59 110.49) (width 0.7) (layer B.Cu) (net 4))
 (segment (start 125.73 110.49) (end 132.08 110.49) (width 0.7) (layer B.Cu) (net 4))
 (segment (start 163.83 104.87) (end 163.83 103.6) (width 0.7) (layer B.Cu) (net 4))
 (segment (start 163.83 110.49) (end 163.83 104.87) (width 0.7) (layer B.Cu) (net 4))
 (segment (start 168.91 110.49) (end 163.83 110.49) (width 0.7) (layer B.Cu) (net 4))
 (segment (start 160.02 110.49) (end 190.5 110.49) (width 0.7) (layer B.Cu) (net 4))
 (segment (start 157.48 110.49) (end 160.02 110.49) (width 0.7) (layer B.Cu) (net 4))
 (segment (start 160.02 106.91) (end 160.02 110.49) (width 0.56) (layer B.Cu) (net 4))
 (segment (start 149.86 105.41) (end 149.86 110.49) (width 0.56) (layer B.Cu) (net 4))
 (segment (start 125.73 60.96) (end 125.73 110.49) (width 0.9) (layer B.Cu) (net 4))
 (segment (start 125.73 110.49) (end 194.31 110.49) (width 0.9) (layer B.Cu) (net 4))
 (segment (start 194.31 110.49) (end 194.31 60.96) (width 0.9) (layer B.Cu) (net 4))
 (segment (start 194.31 60.96) (end 158.75 60.96) (width 0.9) (layer B.Cu) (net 4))
 (segment (start 158.75 60.96) (end 125.73 60.96) (width 0.9) (layer B.Cu) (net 4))
 (segment (start 161.29 60.96) (end 158.75 60.96) (width 0.9) (layer B.Cu) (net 4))
 (segment (start 160.9 69.85) (end 160.9 61.35) (width 0.9) (layer B.Cu) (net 4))
 (segment (start 159.2 74.93) (end 159.2 77.92) (width 0.56) (layer B.Cu) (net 13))
 (segment (start 159.2 77.92) (end 160.02 78.74) (width 0.56) (layer B.Cu) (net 13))
 (segment (start 160.02 88.9) (end 160.02 105.41) (width 0.56) (layer B.Cu) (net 13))
 (segment (start 160.02 78.74) (end 160.02 88.9) (width 0.56) (layer B.Cu) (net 13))
 (segment (start 160.02 88.9) (end 160.02 90.17) (width 0.56) (layer B.Cu) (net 13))
 (segment (start 168.91 91.44) (end 176.54 91.44) (width 0.7) (layer B.Cu) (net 8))
 (segment (start 168.91 99.06) (end 168.91 91.44) (width 0.7) (layer B.Cu) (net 8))
 (segment (start 163.83 99.06) (end 163.83 101.6) (width 0.7) (layer B.Cu) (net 8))
 (segment (start 168.91 99.06) (end 163.83 99.06) (width 0.7) (layer B.Cu) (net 8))
 (segment (start 166 82.92) (end 163.83 85.09) (width 0.7) (layer B.Cu) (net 8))
 (segment (start 166 74.93) (end 166 82.92) (width 0.7) (layer B.Cu) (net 8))
 (segment (start 163.83 85.09) (end 163.83 101.6) (width 0.7) (layer B.Cu) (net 8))
 (segment (start 189.23 73.66) (end 189.23 101.6) (width 0.7) (layer B.Cu) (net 12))
 (segment (start 181.61 73.66) (end 189.23 73.66) (width 0.7) (layer B.Cu) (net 12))
 (segment (start 179.07 69.85) (end 181.61 73.66) (width 0.7) (layer B.Cu) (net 12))
 (segment (start 176.53 72.43) (end 176.53 69.85) (width 0.7) (layer B.Cu) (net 12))
 (segment (start 176.53 69.85) (end 179.07 69.85) (width 0.7) (layer B.Cu) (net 12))
 (segment (start 167.7 69.85) (end 176.53 69.85) (width 0.7) (layer B.Cu) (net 12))
 (segment (start 189.23 101.6) (end 187.96 102.87) (width 0.7) (layer B.Cu) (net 12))
 (segment (start 187.96 102.87) (end 187.96 105.41) (width 0.7) (layer B.Cu) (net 12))
 (segment (start 167.7 69.85) (end 167.7 71.871454) (width 0.56) (layer B.Cu) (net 12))
 (segment (start 167.7 71.871454) (end 166.69052 72.880934) (width 0.56) (layer B.Cu) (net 12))
 (segment (start 166.69052 72.880934) (end 146.922621 72.880934) (width 0.56) (layer B.Cu) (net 12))
 (segment (start 144.78 75.023555) (end 144.78 77.47) (width 0.56) (layer B.Cu) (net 12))
 (segment (start 146.922621 72.880934) (end 144.78 75.023555) (width 0.56) (layer B.Cu) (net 12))
 (segment (start 169.4 74.93) (end 176.53 74.93) (width 0.7) (layer B.Cu) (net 11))
 (segment (start 164.3 65.57) (end 165.1 64.77) (width 0.7) (layer B.Cu) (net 6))
 (segment (start 164.3 69.85) (end 164.3 65.57) (width 0.7) (layer B.Cu) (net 6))
 (segment (start 165.1 64.77) (end 176.53 64.77) (width 0.7) (layer B.Cu) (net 6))
 (segment (start 176.53 64.77) (end 191.77 64.77) (width 0.7) (layer B.Cu) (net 6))
 (segment (start 189.23 71.12) (end 191.77 71.12) (width 0.7) (layer B.Cu) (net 6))
 (segment (start 191.77 71.12) (end 191.77 105.41) (width 0.7) (layer B.Cu) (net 6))
 (segment (start 191.77 64.77) (end 191.77 71.12) (width 0.7) (layer B.Cu) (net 6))
 (segment (start 190.5 107.95) (end 184.15 107.95) (width 0.7) (layer B.Cu) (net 6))
 (segment (start 191.46 106.99) (end 190.5 107.95) (width 0.7) (layer B.Cu) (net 6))
 (segment (start 191.46 105.41) (end 191.46 106.99) (width 0.7) (layer B.Cu) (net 6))
 (segment (start 184.15 107.95) (end 184.15 101.6) (width 0.7) (layer B.Cu) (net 6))
 (segment (start 184.15 101.6) (end 184.15 100.33) (width 0.7) (layer B.Cu) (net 6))
 (segment (start 184.15 82.55) (end 181.57 82.55) (width 0.7) (layer B.Cu) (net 6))
 (segment (start 184.15 101.6) (end 184.15 82.55) (width 0.7) (layer B.Cu) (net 6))
 (segment (start 164.3 69.85) (end 162.32368 71.82632) (width 0.56) (layer B.Cu) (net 6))
 (segment (start 144.07368 71.82632) (end 142.24 73.66) (width 0.56) (layer B.Cu) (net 6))
 (segment (start 162.32368 71.82632) (end 144.07368 71.82632) (width 0.56) (layer B.Cu) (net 6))
 (segment (start 170.18 80.01) (end 176.53 80.01) (width 0.7) (layer B.Cu) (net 2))
 (segment (start 176.53 80.01) (end 179.07 82.55) (width 0.7) (layer B.Cu) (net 2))
 (segment (start 132.08 83.78) (end 132.08 90.17) (width 0.7) (layer B.Cu) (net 5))
 (segment (start 133.31 83.78) (end 132.08 83.78) (width 0.7) (layer B.Cu) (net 5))
 (segment (start 133.35 83.82) (end 133.31 83.78) (width 0.7) (layer B.Cu) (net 5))
 (segment (start 137.16 83.82) (end 133.35 83.82) (width 0.7) (layer B.Cu) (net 5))
 (segment (start 137.16 73.66) (end 137.16 83.82) (width 0.7) (layer B.Cu) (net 5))
 (segment (start 132.08 64.77) (end 132.08 81.28) (width 0.7) (layer B.Cu) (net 14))
 (segment (start 157.48 64.77) (end 132.08 64.77) (width 0.7) (layer B.Cu) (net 14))
 (segment (start 157.5 64.79) (end 157.48 64.77) (width 0.7) (layer B.Cu) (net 14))
 (segment (start 157.5 69.85) (end 157.5 64.79) (width 0.7) (layer B.Cu) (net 14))
 (segment (start 132.08 95.25) (end 132.08 100.33) (width 0.7) (layer B.Cu) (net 17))
 (segment (start 135.89 90.21) (end 137.2 88.9) (width 0.7) (layer B.Cu) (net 17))
 (segment (start 135.89 95.25) (end 135.89 90.21) (width 0.7) (layer B.Cu) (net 17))
 (segment (start 132.08 95.25) (end 134.62 95.25) (width 0.7) (layer B.Cu) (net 17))
 (segment (start 134.62 95.25) (end 135.89 95.25) (width 0.7) (layer B.Cu) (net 17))
 (segment (start 144.78 95.25) (end 144.78 82.55) (width 0.7) (layer B.Cu) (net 17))
 (segment (start 134.62 95.25) (end 144.78 95.25) (width 0.7) (layer B.Cu) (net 17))
 (segment (start 154.1 69.85) (end 139.7 69.85) (width 0.7) (layer B.Cu) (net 15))
 (segment (start 139.7 69.85) (end 139.7 88.9) (width 0.7) (layer B.Cu) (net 15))
 (segment (start 186.69 82.51) (end 186.65 82.55) (width 0.7) (layer B.Cu) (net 10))
 (segment (start 186.69 76.2) (end 186.69 82.51) (width 0.7) (layer B.Cu) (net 10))
 (segment (start 186.73 67.35) (end 186.69 67.31) (width 0.7) (layer B.Cu) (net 9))
 (segment (start 186.73 71.12) (end 186.73 67.35) (width 0.7) (layer B.Cu) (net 9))
 (segment (start 173.99 101.6) (end 173.99 105.41) (width 0.7) (layer B.Cu) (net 18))
 (segment (start 173.99 97.79) (end 173.99 101.6) (width 0.7) (layer B.Cu) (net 18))
 (segment (start 176.53 96.52) (end 173.99 97.79) (width 0.7) (layer B.Cu) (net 18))
 (segment (start 155.8 84.68) (end 156.21 85.09) (width 0.7) (layer B.Cu) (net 7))
 (segment (start 155.8 74.93) (end 155.8 84.68) (width 0.7) (layer B.Cu) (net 7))
 (segment (start 162.56 74.97) (end 162.6 74.93) (width 0.7) (layer B.Cu) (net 1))
 (segment (start 162.56 80.01) (end 162.56 74.97) (width 0.7) (layer B.Cu) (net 1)))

